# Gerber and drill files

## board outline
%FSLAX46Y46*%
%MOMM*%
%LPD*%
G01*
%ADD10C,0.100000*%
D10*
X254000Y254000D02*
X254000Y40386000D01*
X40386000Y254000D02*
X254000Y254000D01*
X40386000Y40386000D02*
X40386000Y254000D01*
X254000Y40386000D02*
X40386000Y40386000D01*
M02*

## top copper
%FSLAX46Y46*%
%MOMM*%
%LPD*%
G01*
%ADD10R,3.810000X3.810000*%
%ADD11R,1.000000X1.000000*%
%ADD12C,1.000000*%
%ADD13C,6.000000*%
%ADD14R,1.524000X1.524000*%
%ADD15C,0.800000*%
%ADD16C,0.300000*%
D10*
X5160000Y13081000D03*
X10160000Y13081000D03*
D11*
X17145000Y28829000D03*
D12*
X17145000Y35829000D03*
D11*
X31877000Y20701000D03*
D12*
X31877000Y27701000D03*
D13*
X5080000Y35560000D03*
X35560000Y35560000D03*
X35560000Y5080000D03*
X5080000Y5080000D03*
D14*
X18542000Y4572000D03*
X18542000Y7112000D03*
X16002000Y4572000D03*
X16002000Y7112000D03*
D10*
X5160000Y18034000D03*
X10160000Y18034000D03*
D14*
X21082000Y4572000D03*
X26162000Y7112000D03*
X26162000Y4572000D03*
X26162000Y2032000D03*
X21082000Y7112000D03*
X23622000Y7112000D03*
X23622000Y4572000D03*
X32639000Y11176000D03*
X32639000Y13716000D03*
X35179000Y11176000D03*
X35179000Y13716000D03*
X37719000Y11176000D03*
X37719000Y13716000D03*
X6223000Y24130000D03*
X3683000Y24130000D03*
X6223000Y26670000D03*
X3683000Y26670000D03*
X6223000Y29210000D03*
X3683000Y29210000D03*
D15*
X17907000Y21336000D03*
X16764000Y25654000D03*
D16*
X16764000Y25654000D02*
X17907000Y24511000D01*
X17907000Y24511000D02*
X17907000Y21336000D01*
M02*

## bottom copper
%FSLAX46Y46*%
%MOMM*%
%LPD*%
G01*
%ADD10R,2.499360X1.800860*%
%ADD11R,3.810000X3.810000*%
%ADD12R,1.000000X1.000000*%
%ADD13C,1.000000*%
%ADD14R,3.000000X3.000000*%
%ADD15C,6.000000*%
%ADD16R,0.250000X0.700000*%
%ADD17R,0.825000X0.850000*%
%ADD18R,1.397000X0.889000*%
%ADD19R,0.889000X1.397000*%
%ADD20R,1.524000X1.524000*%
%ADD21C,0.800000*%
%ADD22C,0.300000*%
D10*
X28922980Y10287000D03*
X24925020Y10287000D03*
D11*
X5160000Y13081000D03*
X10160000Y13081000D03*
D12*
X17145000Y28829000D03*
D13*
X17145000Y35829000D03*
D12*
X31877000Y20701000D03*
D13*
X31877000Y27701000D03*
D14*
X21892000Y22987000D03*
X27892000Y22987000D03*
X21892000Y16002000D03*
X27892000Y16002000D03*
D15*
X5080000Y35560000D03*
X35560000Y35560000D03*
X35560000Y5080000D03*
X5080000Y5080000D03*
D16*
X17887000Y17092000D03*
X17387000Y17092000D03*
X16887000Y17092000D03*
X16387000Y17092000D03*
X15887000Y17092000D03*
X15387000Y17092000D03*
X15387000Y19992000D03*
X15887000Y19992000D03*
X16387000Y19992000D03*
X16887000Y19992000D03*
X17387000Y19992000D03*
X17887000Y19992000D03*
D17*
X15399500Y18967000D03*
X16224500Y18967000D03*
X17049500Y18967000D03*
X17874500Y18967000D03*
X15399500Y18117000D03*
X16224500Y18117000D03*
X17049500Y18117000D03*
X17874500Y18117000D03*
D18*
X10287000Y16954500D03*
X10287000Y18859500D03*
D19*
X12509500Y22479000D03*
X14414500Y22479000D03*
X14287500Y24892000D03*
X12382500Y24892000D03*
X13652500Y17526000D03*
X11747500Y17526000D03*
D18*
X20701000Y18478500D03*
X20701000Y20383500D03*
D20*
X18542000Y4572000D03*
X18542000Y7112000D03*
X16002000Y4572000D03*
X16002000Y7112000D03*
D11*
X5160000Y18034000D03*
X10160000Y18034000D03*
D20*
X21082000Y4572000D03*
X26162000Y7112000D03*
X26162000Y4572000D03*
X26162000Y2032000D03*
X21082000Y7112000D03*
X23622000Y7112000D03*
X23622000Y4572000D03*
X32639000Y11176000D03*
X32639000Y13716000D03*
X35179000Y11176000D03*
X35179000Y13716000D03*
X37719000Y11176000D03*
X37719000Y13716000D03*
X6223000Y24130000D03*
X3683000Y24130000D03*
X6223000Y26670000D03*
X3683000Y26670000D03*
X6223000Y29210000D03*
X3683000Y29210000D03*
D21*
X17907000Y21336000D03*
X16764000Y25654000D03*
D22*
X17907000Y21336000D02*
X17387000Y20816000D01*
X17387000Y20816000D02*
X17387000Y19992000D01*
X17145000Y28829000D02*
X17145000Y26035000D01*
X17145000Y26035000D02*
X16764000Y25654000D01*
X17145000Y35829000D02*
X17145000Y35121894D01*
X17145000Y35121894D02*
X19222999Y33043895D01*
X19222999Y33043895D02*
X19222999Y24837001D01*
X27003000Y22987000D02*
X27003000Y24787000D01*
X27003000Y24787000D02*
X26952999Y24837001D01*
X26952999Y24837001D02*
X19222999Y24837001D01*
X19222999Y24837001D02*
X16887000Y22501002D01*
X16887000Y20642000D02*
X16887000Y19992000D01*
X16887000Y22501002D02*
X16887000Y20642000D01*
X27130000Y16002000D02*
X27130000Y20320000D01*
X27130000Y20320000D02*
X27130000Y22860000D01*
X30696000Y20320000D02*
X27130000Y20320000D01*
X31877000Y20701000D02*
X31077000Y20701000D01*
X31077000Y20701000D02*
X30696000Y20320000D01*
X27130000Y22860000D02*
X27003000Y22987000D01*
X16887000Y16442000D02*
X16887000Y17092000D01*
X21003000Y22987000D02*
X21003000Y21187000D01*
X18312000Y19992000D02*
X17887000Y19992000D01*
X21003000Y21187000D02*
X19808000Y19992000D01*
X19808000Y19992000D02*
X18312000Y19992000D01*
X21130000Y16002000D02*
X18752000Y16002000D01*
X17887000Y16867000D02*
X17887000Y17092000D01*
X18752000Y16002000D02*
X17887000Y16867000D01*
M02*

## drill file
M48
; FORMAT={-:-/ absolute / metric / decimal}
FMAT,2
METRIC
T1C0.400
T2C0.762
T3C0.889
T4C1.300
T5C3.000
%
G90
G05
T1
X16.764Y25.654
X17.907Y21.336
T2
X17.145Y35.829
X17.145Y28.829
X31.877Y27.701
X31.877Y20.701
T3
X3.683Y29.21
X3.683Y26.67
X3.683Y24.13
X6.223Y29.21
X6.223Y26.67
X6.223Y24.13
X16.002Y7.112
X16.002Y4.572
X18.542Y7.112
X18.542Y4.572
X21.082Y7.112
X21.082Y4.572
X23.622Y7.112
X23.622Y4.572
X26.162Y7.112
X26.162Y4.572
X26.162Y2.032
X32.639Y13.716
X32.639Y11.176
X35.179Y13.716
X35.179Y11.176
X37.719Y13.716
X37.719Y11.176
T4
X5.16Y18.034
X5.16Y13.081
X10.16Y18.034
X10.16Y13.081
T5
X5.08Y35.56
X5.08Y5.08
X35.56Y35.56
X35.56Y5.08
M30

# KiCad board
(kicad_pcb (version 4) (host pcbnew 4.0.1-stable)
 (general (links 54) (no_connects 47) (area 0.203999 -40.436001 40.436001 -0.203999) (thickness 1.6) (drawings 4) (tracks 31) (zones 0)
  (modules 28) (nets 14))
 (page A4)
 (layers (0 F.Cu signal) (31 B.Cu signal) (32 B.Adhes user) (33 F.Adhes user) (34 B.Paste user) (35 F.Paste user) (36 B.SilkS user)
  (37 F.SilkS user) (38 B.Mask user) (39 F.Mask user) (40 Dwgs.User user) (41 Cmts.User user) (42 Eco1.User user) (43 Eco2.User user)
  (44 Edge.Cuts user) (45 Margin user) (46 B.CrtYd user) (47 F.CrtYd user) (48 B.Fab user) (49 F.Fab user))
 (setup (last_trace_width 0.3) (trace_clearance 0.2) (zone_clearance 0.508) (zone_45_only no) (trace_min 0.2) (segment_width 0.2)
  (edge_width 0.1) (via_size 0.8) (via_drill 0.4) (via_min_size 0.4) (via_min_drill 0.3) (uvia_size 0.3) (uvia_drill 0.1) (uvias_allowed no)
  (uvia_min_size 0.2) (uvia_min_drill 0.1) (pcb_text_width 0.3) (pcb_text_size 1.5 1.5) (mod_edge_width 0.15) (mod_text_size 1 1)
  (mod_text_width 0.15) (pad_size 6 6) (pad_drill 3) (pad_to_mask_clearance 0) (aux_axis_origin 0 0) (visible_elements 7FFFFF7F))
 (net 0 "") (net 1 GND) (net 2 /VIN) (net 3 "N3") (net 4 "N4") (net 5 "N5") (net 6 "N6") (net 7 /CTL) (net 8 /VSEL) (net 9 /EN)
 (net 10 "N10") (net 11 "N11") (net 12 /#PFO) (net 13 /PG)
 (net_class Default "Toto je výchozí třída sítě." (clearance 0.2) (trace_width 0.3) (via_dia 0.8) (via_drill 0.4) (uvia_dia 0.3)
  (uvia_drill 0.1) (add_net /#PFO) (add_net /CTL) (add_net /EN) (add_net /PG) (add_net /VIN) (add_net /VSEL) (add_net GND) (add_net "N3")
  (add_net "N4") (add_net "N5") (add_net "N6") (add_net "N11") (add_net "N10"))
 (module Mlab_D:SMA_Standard (layer B.Cu) (at 26.924 -10.287 180)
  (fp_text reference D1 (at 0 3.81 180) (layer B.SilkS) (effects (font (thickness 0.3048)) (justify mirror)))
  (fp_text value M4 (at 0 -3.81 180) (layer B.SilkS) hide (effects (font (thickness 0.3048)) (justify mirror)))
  (pad 1 smd rect (at -1.99898 0 180) (size 2.49936 1.80086) (layers B.Cu B.Paste B.Mask) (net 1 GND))
  (pad 2 smd rect (at 1.99898 0 180) (size 2.49936 1.80086) (layers B.Cu B.Paste B.Mask) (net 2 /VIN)))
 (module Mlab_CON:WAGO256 (layer F.Cu) (at 7.62 -13.081)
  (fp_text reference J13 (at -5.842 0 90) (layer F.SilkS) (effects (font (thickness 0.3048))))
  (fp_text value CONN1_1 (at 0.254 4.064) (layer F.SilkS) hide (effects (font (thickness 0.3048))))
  (pad 1 thru_hole rect (at -2.46 0 90) (size 3.81 3.81) (drill 1.3) (layers *.Cu *.Mask F.SilkS) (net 1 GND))
  (pad 1 thru_hole rect (at 2.54 0 90) (size 3.81 3.81) (drill 1.3) (layers *.Cu *.Mask F.SilkS) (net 1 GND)))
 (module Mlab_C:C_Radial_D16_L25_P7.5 (layer F.Cu) (at 17.145 -28.829 90)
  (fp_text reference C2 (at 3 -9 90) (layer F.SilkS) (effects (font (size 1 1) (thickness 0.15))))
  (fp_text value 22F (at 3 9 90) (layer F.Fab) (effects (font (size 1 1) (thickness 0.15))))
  (pad 1 thru_hole rect (at 0 0 90) (size 1 1) (drill 0.762) (layers *.Cu *.Mask F.SilkS) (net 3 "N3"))
  (pad 2 thru_hole circle (at 7 0 90) (size 1 1) (drill 0.762) (layers *.Cu *.Mask F.SilkS) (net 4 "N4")))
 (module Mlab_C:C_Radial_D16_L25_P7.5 (layer F.Cu) (at 31.877 -20.701 90)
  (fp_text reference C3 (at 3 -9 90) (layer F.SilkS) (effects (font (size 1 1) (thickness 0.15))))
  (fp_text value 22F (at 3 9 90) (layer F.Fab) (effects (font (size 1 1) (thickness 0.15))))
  (pad 1 thru_hole rect (at 0 0 90) (size 1 1) (drill 0.762) (layers *.Cu *.Mask F.SilkS) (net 4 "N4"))
  (pad 2 thru_hole circle (at 7 0 90) (size 1 1) (drill 0.762) (layers *.Cu *.Mask F.SilkS) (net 1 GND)))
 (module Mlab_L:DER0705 (layer B.Cu) (at 24.892 -22.987 180)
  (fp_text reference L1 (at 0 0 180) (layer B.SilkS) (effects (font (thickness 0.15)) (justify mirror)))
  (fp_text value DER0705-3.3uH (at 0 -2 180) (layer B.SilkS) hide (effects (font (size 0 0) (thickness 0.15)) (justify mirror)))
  (pad 1 smd rect (at 3 0 180) (size 3 3) (layers B.Cu B.Paste B.Mask) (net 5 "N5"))
  (pad 2 smd rect (at -3 0 180) (size 3 3) (layers B.Cu B.Paste B.Mask) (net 4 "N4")))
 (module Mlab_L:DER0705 (layer B.Cu) (at 24.892 -16.002 180)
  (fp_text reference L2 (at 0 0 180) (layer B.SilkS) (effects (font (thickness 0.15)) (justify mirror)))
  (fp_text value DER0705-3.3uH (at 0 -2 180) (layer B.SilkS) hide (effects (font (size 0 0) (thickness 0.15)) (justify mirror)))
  (pad 1 smd rect (at 3 0 180) (size 3 3) (layers B.Cu B.Paste B.Mask) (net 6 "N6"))
  (pad 2 smd rect (at -3 0 180) (size 3 3) (layers B.Cu B.Paste B.Mask) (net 4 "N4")))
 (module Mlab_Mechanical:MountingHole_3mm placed (layer F.Cu) (at 5.08 -35.56)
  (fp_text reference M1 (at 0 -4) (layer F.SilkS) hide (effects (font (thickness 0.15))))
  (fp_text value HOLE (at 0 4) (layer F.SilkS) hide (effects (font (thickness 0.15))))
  (pad 1 thru_hole circle (at 0 0) (size 6 6) (drill 3) (layers *.Cu *.Adhes *.Mask) (clearance 1) (zone_connect 2)))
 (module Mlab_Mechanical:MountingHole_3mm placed (layer F.Cu) (at 35.56 -35.56)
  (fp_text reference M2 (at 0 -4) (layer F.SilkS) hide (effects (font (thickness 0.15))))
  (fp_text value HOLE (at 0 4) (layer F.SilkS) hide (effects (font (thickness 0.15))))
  (pad 1 thru_hole circle (at 0 0) (size 6 6) (drill 3) (layers *.Cu *.Adhes *.Mask) (clearance 1) (zone_connect 2)))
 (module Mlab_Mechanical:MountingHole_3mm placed (layer F.Cu) (at 35.56 -5.08)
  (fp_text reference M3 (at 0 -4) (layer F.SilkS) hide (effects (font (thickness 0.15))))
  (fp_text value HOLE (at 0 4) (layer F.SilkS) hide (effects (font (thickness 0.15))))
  (pad 1 thru_hole circle (at 0 0) (size 6 6) (drill 3) (layers *.Cu *.Adhes *.Mask) (clearance 1) (zone_connect 2)))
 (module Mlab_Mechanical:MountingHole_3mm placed (layer F.Cu) (at 5.08 -5.08)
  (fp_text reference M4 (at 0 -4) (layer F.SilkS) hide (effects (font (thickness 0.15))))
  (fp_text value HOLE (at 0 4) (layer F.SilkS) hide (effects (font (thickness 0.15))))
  (pad 1 thru_hole circle (at 0 0) (size 6 6) (drill 3) (layers *.Cu *.Adhes *.Mask) (clearance 1) (zone_connect 2)))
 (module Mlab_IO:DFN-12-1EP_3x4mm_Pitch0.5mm (layer B.Cu) (at 16.637 -18.542 90)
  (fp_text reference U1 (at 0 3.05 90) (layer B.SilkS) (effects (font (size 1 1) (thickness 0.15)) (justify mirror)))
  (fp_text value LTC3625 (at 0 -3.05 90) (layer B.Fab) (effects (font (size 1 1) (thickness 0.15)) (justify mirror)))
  (pad 1 smd rect (at -1.45 1.25 90) (size 0.7 0.25) (layers B.Cu B.Paste B.Mask) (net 6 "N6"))
  (pad 2 smd rect (at -1.45 0.75 90) (size 0.7 0.25) (layers B.Cu B.Paste B.Mask) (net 2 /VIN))
  (pad 3 smd rect (at -1.45 0.25 90) (size 0.7 0.25) (layers B.Cu B.Paste B.Mask) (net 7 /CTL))
  (pad 4 smd rect (at -1.45 -0.25 90) (size 0.7 0.25) (layers B.Cu B.Paste B.Mask) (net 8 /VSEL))
  (pad 5 smd rect (at -1.45 -0.75 90) (size 0.7 0.25) (layers B.Cu B.Paste B.Mask) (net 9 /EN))
  (pad 6 smd rect (at -1.45 -1.25 90) (size 0.7 0.25) (layers B.Cu B.Paste B.Mask) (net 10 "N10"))
  (pad 7 smd rect (at 1.45 -1.25 90) (size 0.7 0.25) (layers B.Cu B.Paste B.Mask) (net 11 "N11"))
  (pad 8 smd rect (at 1.45 -0.75 90) (size 0.7 0.25) (layers B.Cu B.Paste B.Mask) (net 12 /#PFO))
  (pad 9 smd rect (at 1.45 -0.25 90) (size 0.7 0.25) (layers B.Cu B.Paste B.Mask) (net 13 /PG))
  (pad 10 smd rect (at 1.45 0.25 90) (size 0.7 0.25) (layers B.Cu B.Paste B.Mask) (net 4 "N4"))
  (pad 11 smd rect (at 1.45 0.75 90) (size 0.7 0.25) (layers B.Cu B.Paste B.Mask) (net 3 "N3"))
  (pad 12 smd rect (at 1.45 1.25 90) (size 0.7 0.25) (layers B.Cu B.Paste B.Mask) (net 5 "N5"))
  (pad 13 smd rect (at 0.425 -1.2375 90) (size 0.85 0.825) (layers B.Cu B.Paste B.Mask) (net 1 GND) (solder_paste_margin_ratio -0.2))
  (pad 13 smd rect (at 0.425 -0.4125 90) (size 0.85 0.825) (layers B.Cu B.Paste B.Mask) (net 1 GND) (solder_paste_margin_ratio -0.2))
  (pad 13 smd rect (at 0.425 0.4125 90) (size 0.85 0.825) (layers B.Cu B.Paste B.Mask) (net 1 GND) (solder_paste_margin_ratio -0.2))
  (pad 13 smd rect (at 0.425 1.2375 90) (size 0.85 0.825) (layers B.Cu B.Paste B.Mask) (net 1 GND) (solder_paste_margin_ratio -0.2))
  (pad 13 smd rect (at -0.425 -1.2375 90) (size 0.85 0.825) (layers B.Cu B.Paste B.Mask) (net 1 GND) (solder_paste_margin_ratio -0.2))
  (pad 13 smd rect (at -0.425 -0.4125 90) (size 0.85 0.825) (layers B.Cu B.Paste B.Mask) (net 1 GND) (solder_paste_margin_ratio -0.2))
  (pad 13 smd rect (at -0.425 0.4125 90) (size 0.85 0.825) (layers B.Cu B.Paste B.Mask) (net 1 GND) (solder_paste_margin_ratio -0.2))
  (pad 13 smd rect (at -0.425 1.2375 90) (size 0.85 0.825) (layers B.Cu B.Paste B.Mask) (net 1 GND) (solder_paste_margin_ratio -0.2)))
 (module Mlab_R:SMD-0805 (layer B.Cu) (at 10.287 -17.907 90)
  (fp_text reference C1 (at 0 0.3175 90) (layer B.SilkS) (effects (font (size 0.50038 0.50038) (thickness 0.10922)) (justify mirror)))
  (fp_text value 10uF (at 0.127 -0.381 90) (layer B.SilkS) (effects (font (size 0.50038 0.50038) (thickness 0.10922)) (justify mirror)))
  (pad 1 smd rect (at -0.9525 0 90) (size 0.889 1.397) (layers B.Cu B.Paste B.Mask) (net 2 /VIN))
  (pad 2 smd rect (at 0.9525 0 90) (size 0.889 1.397) (layers B.Cu B.Paste B.Mask) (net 1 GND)))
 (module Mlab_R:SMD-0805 (layer B.Cu) (at 13.462 -22.479)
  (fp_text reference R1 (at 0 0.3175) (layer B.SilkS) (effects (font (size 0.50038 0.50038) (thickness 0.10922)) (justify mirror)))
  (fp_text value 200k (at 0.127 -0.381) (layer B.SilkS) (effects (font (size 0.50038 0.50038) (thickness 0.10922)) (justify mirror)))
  (pad 1 smd rect (at -0.9525 0) (size 0.889 1.397) (layers B.Cu B.Paste B.Mask) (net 2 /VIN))
  (pad 2 smd rect (at 0.9525 0) (size 0.889 1.397) (layers B.Cu B.Paste B.Mask) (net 11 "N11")))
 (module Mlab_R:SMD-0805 (layer B.Cu) (at 13.335 -24.892 180)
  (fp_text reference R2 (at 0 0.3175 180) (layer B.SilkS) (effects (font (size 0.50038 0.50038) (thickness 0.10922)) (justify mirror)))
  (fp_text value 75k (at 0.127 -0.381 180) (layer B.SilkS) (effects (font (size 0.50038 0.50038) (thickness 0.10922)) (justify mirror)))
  (pad 1 smd rect (at -0.9525 0 180) (size 0.889 1.397) (layers B.Cu B.Paste B.Mask) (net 11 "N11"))
  (pad 2 smd rect (at 0.9525 0 180) (size 0.889 1.397) (layers B.Cu B.Paste B.Mask) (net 1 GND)))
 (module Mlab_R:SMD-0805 (layer B.Cu) (at 12.7 -17.526 180)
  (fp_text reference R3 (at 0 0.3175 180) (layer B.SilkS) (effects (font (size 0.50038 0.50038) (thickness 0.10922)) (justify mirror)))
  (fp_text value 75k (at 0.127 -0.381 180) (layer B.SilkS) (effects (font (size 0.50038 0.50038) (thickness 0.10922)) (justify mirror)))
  (pad 1 smd rect (at -0.9525 0 180) (size 0.889 1.397) (layers B.Cu B.Paste B.Mask) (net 10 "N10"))
  (pad 2 smd rect (at 0.9525 0 180) (size 0.889 1.397) (layers B.Cu B.Paste B.Mask) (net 1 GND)))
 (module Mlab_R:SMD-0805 (layer B.Cu) (at 20.701 -19.431 90)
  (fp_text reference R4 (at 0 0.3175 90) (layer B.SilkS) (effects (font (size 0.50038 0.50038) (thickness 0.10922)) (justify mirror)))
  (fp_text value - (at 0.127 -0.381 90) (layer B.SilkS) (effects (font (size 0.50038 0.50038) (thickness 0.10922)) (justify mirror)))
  (pad 1 smd rect (at -0.9525 0 90) (size 0.889 1.397) (layers B.Cu B.Paste B.Mask) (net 5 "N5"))
  (pad 2 smd rect (at 0.9525 0 90) (size 0.889 1.397) (layers B.Cu B.Paste B.Mask) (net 6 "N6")))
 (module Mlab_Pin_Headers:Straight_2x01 (layer F.Cu) (at 18.542 -5.842 90)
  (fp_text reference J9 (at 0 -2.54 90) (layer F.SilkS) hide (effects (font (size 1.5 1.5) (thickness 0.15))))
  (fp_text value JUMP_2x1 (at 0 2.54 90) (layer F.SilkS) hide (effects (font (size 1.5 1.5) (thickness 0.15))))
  (pad 1 thru_hole rect (at -1.27 0 90) (size 1.524 1.524) (drill 0.889) (layers *.Cu *.Mask F.SilkS) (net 12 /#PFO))
  (pad 2 thru_hole rect (at 1.27 0 90) (size 1.524 1.524) (drill 0.889) (layers *.Cu *.Mask F.SilkS) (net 12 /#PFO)))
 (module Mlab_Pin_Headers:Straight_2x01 (layer F.Cu) (at 16.002 -5.842 90)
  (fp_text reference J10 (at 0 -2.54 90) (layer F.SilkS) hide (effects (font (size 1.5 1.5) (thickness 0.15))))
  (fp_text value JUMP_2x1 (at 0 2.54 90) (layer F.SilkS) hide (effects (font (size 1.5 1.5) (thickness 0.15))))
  (pad 1 thru_hole rect (at -1.27 0 90) (size 1.524 1.524) (drill 0.889) (layers *.Cu *.Mask F.SilkS) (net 13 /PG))
  (pad 2 thru_hole rect (at 1.27 0 90) (size 1.524 1.524) (drill 0.889) (layers *.Cu *.Mask F.SilkS) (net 13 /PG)))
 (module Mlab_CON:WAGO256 (layer F.Cu) (at 7.62 -18.034)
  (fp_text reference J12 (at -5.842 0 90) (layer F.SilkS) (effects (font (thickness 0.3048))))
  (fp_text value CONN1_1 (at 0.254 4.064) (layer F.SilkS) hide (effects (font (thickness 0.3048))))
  (pad 1 thru_hole rect (at -2.46 0 90) (size 3.81 3.81) (drill 1.3) (layers *.Cu *.Mask F.SilkS) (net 3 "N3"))
  (pad 1 thru_hole rect (at 2.54 0 90) (size 3.81 3.81) (drill 1.3) (layers *.Cu *.Mask F.SilkS) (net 3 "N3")))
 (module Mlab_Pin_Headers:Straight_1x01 (layer F.Cu) (at 21.082 -4.572)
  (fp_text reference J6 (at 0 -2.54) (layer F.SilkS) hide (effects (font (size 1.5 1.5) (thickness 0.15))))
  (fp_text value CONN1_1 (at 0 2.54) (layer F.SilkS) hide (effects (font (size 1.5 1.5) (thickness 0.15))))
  (pad 1 thru_hole rect (at 0 0) (size 1.524 1.524) (drill 0.889) (layers *.Cu *.Mask F.SilkS) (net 9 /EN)))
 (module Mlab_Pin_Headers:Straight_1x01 (layer F.Cu) (at 26.162 -7.112)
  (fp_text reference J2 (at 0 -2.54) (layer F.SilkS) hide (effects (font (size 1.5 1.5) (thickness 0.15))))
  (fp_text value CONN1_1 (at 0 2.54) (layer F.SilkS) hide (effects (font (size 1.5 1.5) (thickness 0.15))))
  (pad 1 thru_hole rect (at 0 0) (size 1.524 1.524) (drill 0.889) (layers *.Cu *.Mask F.SilkS) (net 2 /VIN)))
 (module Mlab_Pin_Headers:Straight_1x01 (layer F.Cu) (at 26.162 -4.572)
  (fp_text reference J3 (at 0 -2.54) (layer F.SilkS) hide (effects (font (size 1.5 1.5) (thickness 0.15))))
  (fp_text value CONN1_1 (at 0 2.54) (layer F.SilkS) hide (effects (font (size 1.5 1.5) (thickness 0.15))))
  (pad 1 thru_hole rect (at 0 0) (size 1.524 1.524) (drill 0.889) (layers *.Cu *.Mask F.SilkS) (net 7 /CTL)))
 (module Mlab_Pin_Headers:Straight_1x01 (layer F.Cu) (at 26.162 -2.032)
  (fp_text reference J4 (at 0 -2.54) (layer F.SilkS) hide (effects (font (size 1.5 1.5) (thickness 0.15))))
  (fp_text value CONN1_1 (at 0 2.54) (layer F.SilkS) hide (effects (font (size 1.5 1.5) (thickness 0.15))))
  (pad 1 thru_hole rect (at 0 0) (size 1.524 1.524) (drill 0.889) (layers *.Cu *.Mask F.SilkS) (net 1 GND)))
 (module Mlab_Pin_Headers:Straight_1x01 (layer F.Cu) (at 21.082 -7.112)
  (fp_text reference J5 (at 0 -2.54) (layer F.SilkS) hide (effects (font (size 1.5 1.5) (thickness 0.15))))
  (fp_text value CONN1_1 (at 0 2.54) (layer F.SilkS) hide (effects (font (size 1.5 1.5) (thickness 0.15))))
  (pad 1 thru_hole rect (at 0 0) (size 1.524 1.524) (drill 0.889) (layers *.Cu *.Mask F.SilkS) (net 2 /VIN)))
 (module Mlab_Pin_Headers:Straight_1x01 (layer F.Cu) (at 23.622 -7.112)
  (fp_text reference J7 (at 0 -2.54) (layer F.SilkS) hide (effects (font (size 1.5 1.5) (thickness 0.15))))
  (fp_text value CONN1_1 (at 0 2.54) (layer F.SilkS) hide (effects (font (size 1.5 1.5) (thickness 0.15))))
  (pad 1 thru_hole rect (at 0 0) (size 1.524 1.524) (drill 0.889) (layers *.Cu *.Mask F.SilkS) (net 2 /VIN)))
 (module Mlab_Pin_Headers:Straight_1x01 (layer F.Cu) (at 23.622 -4.572)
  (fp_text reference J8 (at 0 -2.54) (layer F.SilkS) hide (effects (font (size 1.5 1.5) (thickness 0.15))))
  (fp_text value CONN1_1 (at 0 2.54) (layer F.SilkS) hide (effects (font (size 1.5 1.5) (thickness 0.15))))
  (pad 1 thru_hole rect (at 0 0) (size 1.524 1.524) (drill 0.889) (layers *.Cu *.Mask F.SilkS) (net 8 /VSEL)))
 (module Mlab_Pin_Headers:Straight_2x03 (layer F.Cu) (at 35.179 -12.446 90)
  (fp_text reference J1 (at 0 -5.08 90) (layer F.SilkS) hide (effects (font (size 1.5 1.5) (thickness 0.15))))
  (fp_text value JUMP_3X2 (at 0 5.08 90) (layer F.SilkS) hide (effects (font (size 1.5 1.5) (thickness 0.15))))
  (pad 1 thru_hole rect (at -1.27 -2.54 90) (size 1.524 1.524) (drill 0.889) (layers *.Cu *.Mask F.SilkS) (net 1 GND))
  (pad 2 thru_hole rect (at 1.27 -2.54 90) (size 1.524 1.524) (drill 0.889) (layers *.Cu *.Mask F.SilkS) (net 1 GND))
  (pad 3 thru_hole rect (at -1.27 0 90) (size 1.524 1.524) (drill 0.889) (layers *.Cu *.Mask F.SilkS) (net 2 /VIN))
  (pad 4 thru_hole rect (at 1.27 0 90) (size 1.524 1.524) (drill 0.889) (layers *.Cu *.Mask F.SilkS) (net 2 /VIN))
  (pad 5 thru_hole rect (at -1.27 2.54 90) (size 1.524 1.524) (drill 0.889) (layers *.Cu *.Mask F.SilkS) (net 1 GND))
  (pad 6 thru_hole rect (at 1.27 2.54 90) (size 1.524 1.524) (drill 0.889) (layers *.Cu *.Mask F.SilkS) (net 1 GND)))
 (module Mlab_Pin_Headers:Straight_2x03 (layer F.Cu) (at 4.953 -26.67 180)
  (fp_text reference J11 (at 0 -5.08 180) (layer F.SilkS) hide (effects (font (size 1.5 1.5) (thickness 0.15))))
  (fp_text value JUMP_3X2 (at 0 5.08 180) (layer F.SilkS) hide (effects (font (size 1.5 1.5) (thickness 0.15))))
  (pad 1 thru_hole rect (at -1.27 -2.54 180) (size 1.524 1.524) (drill 0.889) (layers *.Cu *.Mask F.SilkS) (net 1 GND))
  (pad 2 thru_hole rect (at 1.27 -2.54 180) (size 1.524 1.524) (drill 0.889) (layers *.Cu *.Mask F.SilkS) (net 1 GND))
  (pad 3 thru_hole rect (at -1.27 0 180) (size 1.524 1.524) (drill 0.889) (layers *.Cu *.Mask F.SilkS) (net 3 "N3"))
  (pad 4 thru_hole rect (at 1.27 0 180) (size 1.524 1.524) (drill 0.889) (layers *.Cu *.Mask F.SilkS) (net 3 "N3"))
  (pad 5 thru_hole rect (at -1.27 2.54 180) (size 1.524 1.524) (drill 0.889) (layers *.Cu *.Mask F.SilkS) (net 1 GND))
  (pad 6 thru_hole rect (at 1.27 2.54 180) (size 1.524 1.524) (drill 0.889) (layers *.Cu *.Mask F.SilkS) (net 1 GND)))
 (gr_line (start 0.254 -0.254) (end 0.254 -40.386) (angle 90) (layer Edge.Cuts) (width 0.1))
 (gr_line (start 40.386 -0.254) (end 0.254 -0.254) (angle 90) (layer Edge.Cuts) (width 0.1))
 (gr_line (start 40.386 -40.386) (end 40.386 -0.254) (angle 90) (layer Edge.Cuts) (width 0.1))
 (gr_line (start 0.254 -40.386) (end 40.386 -40.386) (angle 90) (layer Edge.Cuts) (width 0.1))
 (segment (start 17.907 -21.336) (end 17.387 -20.816) (width 0.3) (layer B.Cu) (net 3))
 (segment (start 17.387 -20.816) (end 17.387 -19.992) (width 0.3) (layer B.Cu) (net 3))
 (segment (start 16.764 -25.654) (end 17.907 -24.511) (width 0.3) (layer F.Cu) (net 3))
 (segment (start 17.907 -24.511) (end 17.907 -21.336) (width 0.3) (layer F.Cu) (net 3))
 (via (at 17.907 -21.336) (size 0.8) (drill 0.4) (layers F.Cu B.Cu) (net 3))
 (segment (start 17.145 -28.829) (end 17.145 -26.035) (width 0.3) (layer B.Cu) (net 3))
 (segment (start 17.145 -26.035) (end 16.764 -25.654) (width 0.3) (layer B.Cu) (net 3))
 (via (at 16.764 -25.654) (size 0.8) (drill 0.4) (layers F.Cu B.Cu) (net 3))
 (segment (start 17.145 -35.829) (end 17.145 -35.121894) (width 0.3) (layer B.Cu) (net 4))
 (segment (start 17.145 -35.121894) (end 19.222999 -33.043895) (width 0.3) (layer B.Cu) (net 4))
 (segment (start 19.222999 -33.043895) (end 19.222999 -24.837001) (width 0.3) (layer B.Cu) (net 4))
 (segment (start 27.003 -22.987) (end 27.003 -24.787) (width 0.3) (layer B.Cu) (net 4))
 (segment (start 27.003 -24.787) (end 26.952999 -24.837001) (width 0.3) (layer B.Cu) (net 4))
 (segment (start 26.952999 -24.837001) (end 19.222999 -24.837001) (width 0.3) (layer B.Cu) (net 4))
 (segment (start 19.222999 -24.837001) (end 16.887 -22.501002) (width 0.3) (layer B.Cu) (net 4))
 (segment (start 16.887 -20.642) (end 16.887 -19.992) (width 0.3) (layer B.Cu) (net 4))
 (segment (start 16.887 -22.501002) (end 16.887 -20.642) (width 0.3) (layer B.Cu) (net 4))
 (segment (start 27.13 -16.002) (end 27.13 -20.32) (width 0.3) (layer B.Cu) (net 4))
 (segment (start 27.13 -20.32) (end 27.13 -22.86) (width 0.3) (layer B.Cu) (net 4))
 (segment (start 30.696 -20.32) (end 27.13 -20.32) (width 0.3) (layer B.Cu) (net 4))
 (segment (start 31.877 -20.701) (end 31.077 -20.701) (width 0.3) (layer B.Cu) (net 4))
 (segment (start 31.077 -20.701) (end 30.696 -20.32) (width 0.3) (layer B.Cu) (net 4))
 (segment (start 27.13 -22.86) (end 27.003 -22.987) (width 0.3) (layer B.Cu) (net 4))
 (segment (start 16.887 -16.442) (end 16.887 -17.092) (width 0.3) (layer B.Cu) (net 7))
 (segment (start 21.003 -22.987) (end 21.003 -21.187) (width 0.3) (layer B.Cu) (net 5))
 (segment (start 18.312 -19.992) (end 17.887 -19.992) (width 0.3) (layer B.Cu) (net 5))
 (segment (start 21.003 -21.187) (end 19.808 -19.992) (width 0.3) (layer B.Cu) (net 5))
 (segment (start 19.808 -19.992) (end 18.312 -19.992) (width 0.3) (layer B.Cu) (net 5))
 (segment (start 21.13 -16.002) (end 18.752 -16.002) (width 0.3) (layer B.Cu) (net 6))
 (segment (start 17.887 -16.867) (end 17.887 -17.092) (width 0.3) (layer B.Cu) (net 6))
 (segment (start 18.752 -16.002) (end 17.887 -16.867) (width 0.3) (layer B.Cu) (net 6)))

